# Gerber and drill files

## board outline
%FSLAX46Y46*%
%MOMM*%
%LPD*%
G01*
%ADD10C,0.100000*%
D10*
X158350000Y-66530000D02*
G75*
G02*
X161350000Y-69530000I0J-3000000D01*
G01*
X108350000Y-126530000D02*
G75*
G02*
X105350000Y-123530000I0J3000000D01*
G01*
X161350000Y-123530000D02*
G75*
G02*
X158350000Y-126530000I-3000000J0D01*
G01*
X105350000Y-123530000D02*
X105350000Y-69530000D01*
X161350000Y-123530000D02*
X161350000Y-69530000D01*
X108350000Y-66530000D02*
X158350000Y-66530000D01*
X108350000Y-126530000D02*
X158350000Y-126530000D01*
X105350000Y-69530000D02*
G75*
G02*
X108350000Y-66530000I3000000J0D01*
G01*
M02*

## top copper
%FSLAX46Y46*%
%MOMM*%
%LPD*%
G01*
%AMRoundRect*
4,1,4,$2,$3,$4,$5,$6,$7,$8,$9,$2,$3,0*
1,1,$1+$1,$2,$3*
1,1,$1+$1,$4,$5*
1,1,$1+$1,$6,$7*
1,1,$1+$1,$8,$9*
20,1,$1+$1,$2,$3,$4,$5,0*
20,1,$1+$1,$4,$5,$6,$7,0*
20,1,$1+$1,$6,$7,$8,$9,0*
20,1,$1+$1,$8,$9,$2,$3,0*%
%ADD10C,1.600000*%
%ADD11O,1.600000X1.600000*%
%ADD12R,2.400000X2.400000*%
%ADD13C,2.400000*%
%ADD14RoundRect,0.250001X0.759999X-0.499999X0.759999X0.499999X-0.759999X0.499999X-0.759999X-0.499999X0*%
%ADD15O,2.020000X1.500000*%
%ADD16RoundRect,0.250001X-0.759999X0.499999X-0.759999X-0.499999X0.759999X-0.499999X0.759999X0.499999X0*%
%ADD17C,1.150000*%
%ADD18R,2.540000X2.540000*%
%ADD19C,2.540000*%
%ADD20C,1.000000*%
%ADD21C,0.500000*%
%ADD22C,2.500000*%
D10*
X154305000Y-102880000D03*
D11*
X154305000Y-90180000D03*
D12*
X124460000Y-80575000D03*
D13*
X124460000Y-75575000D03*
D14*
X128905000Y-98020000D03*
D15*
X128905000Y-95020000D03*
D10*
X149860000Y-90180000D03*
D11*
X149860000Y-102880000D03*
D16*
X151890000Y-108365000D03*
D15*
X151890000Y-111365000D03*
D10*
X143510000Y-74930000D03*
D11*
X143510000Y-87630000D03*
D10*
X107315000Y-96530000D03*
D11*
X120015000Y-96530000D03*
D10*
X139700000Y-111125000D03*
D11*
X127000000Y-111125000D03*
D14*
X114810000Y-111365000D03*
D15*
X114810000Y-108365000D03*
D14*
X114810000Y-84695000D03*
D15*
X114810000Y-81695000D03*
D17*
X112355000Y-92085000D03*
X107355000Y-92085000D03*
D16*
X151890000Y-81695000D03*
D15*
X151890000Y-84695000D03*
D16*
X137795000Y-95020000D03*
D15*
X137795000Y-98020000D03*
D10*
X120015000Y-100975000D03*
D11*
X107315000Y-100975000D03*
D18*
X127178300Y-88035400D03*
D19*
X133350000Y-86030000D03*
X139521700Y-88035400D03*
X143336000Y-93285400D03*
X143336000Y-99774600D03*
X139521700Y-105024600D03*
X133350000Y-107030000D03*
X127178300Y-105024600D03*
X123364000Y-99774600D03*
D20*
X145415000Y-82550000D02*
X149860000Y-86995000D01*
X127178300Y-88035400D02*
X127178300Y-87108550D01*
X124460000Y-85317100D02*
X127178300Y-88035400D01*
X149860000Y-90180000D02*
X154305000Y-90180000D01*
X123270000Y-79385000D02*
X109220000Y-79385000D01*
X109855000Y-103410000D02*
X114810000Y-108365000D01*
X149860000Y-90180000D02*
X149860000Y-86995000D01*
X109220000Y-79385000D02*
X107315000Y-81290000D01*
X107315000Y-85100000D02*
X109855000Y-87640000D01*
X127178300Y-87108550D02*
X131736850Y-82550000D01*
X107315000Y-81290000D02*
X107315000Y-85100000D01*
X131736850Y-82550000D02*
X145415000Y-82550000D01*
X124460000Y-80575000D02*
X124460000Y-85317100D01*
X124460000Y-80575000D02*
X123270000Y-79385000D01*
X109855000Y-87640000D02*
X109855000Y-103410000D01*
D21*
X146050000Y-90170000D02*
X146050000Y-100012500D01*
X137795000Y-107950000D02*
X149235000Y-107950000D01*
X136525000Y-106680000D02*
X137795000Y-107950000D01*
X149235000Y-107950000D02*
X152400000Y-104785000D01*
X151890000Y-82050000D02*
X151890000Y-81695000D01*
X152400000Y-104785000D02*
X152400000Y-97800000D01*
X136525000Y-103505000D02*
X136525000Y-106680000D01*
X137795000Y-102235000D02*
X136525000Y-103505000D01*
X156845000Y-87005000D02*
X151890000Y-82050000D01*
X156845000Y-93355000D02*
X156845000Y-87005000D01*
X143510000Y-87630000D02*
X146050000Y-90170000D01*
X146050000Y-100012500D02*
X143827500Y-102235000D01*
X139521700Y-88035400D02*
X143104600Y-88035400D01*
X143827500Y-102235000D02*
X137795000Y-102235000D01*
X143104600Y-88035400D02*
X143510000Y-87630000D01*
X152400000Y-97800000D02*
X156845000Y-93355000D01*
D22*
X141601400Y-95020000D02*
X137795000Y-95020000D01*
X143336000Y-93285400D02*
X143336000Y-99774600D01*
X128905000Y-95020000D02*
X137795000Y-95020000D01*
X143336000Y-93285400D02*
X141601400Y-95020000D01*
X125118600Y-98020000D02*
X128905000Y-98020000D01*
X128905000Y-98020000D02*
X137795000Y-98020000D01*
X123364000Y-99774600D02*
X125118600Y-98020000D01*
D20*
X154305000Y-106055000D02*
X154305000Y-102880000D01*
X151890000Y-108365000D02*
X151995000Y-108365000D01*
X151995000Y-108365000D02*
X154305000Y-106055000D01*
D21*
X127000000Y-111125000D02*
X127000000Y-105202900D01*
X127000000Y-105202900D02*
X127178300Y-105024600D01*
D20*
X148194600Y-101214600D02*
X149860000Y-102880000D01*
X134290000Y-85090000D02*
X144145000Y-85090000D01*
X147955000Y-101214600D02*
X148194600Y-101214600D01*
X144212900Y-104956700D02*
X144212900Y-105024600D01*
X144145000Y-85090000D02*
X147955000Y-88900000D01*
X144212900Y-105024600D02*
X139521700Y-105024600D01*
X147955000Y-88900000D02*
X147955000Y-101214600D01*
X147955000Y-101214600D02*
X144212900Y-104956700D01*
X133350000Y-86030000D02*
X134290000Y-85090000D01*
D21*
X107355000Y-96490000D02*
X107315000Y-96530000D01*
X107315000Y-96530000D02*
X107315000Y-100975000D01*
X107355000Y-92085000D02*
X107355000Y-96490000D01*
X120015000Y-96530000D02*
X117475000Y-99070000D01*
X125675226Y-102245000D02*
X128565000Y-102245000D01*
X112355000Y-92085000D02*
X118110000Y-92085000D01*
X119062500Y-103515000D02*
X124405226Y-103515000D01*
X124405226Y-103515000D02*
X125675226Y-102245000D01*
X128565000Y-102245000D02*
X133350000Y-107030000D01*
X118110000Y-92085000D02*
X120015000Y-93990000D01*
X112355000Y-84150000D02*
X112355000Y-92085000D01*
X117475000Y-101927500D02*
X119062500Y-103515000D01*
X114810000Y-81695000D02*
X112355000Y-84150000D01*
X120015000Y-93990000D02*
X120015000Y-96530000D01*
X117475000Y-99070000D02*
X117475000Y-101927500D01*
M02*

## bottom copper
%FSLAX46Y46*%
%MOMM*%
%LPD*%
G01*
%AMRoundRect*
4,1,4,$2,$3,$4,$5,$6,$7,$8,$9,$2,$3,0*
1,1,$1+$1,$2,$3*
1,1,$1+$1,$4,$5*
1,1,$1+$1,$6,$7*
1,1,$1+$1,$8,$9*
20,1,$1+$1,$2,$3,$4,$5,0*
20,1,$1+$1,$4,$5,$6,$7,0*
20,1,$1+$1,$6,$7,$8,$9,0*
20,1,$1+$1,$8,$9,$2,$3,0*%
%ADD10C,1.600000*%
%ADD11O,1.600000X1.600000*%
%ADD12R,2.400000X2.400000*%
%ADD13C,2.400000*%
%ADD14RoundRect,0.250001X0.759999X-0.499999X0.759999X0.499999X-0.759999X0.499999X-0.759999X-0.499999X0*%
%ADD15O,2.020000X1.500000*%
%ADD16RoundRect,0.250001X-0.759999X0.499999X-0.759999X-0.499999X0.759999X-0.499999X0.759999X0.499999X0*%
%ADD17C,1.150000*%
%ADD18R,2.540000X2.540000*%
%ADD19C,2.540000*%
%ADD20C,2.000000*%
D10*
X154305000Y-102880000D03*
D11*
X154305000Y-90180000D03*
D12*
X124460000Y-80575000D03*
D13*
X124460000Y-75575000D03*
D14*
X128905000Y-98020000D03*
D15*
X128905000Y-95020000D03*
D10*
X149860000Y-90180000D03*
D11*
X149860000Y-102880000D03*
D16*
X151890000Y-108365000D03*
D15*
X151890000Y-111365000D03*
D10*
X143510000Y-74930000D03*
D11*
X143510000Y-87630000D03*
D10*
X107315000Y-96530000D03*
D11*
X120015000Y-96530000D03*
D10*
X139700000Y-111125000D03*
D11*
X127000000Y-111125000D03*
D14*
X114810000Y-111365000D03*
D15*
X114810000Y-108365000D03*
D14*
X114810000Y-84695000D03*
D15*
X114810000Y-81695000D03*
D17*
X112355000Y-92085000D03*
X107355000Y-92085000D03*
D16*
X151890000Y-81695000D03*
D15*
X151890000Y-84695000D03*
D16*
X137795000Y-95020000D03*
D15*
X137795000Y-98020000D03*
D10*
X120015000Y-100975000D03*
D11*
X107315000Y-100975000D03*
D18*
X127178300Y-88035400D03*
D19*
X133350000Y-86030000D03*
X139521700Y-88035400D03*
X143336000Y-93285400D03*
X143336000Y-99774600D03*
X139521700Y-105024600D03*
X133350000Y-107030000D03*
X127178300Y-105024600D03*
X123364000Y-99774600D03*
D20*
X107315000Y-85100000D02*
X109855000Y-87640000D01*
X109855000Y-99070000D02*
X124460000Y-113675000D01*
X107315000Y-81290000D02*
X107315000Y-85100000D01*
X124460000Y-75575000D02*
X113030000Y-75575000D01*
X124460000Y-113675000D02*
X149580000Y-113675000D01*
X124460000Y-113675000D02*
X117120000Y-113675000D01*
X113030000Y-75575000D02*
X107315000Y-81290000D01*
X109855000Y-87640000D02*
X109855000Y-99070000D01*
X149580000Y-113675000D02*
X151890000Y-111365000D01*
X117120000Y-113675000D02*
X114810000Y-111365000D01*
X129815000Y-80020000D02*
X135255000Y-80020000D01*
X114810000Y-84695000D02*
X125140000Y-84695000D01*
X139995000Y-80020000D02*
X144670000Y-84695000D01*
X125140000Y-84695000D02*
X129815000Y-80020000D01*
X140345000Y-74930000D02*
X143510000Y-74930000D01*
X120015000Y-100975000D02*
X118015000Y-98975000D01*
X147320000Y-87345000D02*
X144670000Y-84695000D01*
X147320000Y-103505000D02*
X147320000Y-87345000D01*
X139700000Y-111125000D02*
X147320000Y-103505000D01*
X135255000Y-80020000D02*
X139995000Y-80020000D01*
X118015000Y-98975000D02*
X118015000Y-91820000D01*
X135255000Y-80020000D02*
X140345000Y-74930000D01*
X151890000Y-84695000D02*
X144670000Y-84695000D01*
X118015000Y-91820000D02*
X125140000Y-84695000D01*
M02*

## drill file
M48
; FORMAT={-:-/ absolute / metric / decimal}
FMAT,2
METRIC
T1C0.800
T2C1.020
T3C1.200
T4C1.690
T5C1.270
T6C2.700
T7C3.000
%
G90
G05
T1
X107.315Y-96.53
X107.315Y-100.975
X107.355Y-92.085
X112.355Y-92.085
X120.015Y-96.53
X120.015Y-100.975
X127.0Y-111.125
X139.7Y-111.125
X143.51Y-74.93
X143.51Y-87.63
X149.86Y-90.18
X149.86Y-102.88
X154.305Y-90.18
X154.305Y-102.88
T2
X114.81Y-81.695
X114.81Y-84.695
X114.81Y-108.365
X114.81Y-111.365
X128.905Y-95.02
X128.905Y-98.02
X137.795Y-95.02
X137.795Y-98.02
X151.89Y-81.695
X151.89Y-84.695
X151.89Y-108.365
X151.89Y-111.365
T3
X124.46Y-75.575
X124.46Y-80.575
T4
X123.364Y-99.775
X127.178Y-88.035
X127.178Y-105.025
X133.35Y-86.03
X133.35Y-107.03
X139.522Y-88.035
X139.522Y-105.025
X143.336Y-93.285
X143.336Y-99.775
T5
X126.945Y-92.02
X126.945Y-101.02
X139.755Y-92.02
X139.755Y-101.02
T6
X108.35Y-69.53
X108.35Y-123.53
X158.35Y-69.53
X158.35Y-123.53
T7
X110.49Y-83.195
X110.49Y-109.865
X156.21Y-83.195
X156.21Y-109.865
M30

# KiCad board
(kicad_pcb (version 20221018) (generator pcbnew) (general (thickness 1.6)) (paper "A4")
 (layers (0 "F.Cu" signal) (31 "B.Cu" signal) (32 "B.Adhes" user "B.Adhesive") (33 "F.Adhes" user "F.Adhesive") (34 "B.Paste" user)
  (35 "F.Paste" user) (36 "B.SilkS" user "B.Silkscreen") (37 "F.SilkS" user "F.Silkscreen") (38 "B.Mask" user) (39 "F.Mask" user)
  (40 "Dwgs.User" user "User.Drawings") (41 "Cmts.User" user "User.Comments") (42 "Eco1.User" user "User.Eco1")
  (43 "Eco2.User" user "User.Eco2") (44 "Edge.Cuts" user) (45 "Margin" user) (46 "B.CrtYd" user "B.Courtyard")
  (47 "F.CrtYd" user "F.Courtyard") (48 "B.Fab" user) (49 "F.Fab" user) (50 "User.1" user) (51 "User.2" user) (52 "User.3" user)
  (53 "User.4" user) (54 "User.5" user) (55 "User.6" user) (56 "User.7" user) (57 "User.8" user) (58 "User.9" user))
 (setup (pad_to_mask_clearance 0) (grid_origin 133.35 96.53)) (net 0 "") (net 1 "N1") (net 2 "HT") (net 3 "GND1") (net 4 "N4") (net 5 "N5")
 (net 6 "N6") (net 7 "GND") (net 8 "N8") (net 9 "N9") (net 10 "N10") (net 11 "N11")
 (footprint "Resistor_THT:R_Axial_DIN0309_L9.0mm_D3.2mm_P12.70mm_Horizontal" (layer "F.Cu") (at 154.305 102.88 90)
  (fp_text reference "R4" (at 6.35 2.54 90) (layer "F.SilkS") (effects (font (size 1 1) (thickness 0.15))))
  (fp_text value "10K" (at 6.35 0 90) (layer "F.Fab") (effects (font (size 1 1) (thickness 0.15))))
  (pad "1" thru_hole circle (at 0 0 90) (size 1.6 1.6) (drill 0.8) (layers "*.Cu" "*.Mask") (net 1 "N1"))
  (pad "2" thru_hole oval (at 12.7 0 90) (size 1.6 1.6) (drill 0.8) (layers "*.Cu" "*.Mask") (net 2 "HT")))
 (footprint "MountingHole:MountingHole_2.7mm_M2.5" (layer "F.Cu") (at 158.35 69.53)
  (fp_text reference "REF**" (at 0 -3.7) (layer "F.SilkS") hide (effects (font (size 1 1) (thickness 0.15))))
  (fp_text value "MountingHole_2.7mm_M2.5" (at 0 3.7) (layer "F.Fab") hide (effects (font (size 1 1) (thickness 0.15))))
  (pad "" np_thru_hole circle (at 0 0) (size 2.7 2.7) (drill 2.7) (layers "*.Cu" "*.Mask")))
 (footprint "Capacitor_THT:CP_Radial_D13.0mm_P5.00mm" (layer "F.Cu") (at 124.46 80.575 90)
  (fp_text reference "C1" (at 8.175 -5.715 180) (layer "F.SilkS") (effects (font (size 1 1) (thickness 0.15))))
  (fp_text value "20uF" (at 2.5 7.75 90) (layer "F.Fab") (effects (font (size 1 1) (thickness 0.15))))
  (pad "1" thru_hole rect (at 0 0 90) (size 2.4 2.4) (drill 1.2) (layers "*.Cu" "*.Mask") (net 2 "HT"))
  (pad "2" thru_hole circle (at 5 0 90) (size 2.4 2.4) (drill 1.2) (layers "*.Cu" "*.Mask") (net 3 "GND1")))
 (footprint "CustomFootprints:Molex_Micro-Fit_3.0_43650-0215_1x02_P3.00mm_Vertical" (layer "F.Cu") (at 128.905 98.02 90)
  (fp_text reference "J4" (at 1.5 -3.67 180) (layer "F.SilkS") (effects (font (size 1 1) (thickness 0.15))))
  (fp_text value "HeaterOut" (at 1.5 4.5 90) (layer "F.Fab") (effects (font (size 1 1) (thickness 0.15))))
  (pad "" np_thru_hole circle (at -3 -1.96 90) (size 1.27 1.27) (drill 1.27) (layers "*.Cu" "*.Mask"))
  (pad "" np_thru_hole circle (at 6 -1.96 90) (size 1.27 1.27) (drill 1.27) (layers "*.Cu" "*.Mask"))
  (pad "1" thru_hole roundrect (at 0 0 90) (size 1.5 2.02) (drill 1.02) (layers "*.Cu" "*.Mask") (roundrect_rratio 0.166667) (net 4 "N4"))
  (pad "2" thru_hole oval (at 3 0 90) (size 1.5 2.02) (drill 1.02) (layers "*.Cu" "*.Mask") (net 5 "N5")))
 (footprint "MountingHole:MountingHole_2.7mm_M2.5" (layer "F.Cu") (at 108.35 123.53)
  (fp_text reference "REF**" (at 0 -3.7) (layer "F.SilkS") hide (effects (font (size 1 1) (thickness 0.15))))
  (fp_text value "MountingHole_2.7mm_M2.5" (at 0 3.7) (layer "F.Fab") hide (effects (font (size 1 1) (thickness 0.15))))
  (pad "" np_thru_hole circle (at 0 0) (size 2.7 2.7) (drill 2.7) (layers "*.Cu" "*.Mask")))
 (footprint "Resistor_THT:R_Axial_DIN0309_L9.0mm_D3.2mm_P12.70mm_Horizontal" (layer "F.Cu") (at 149.86 90.18 -90)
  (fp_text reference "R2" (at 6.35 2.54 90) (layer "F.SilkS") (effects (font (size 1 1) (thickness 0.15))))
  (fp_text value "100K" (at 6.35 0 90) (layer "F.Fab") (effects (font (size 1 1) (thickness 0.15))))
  (pad "1" thru_hole circle (at 0 0 270) (size 1.6 1.6) (drill 0.8) (layers "*.Cu" "*.Mask") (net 2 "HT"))
  (pad "2" thru_hole oval (at 12.7 0 270) (size 1.6 1.6) (drill 0.8) (layers "*.Cu" "*.Mask") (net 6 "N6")))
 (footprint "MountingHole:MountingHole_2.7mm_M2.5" (layer "F.Cu") (at 158.35 123.53)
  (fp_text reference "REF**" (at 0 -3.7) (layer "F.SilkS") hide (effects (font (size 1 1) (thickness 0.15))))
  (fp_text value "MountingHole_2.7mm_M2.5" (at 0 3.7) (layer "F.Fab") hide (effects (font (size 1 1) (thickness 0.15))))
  (pad "" np_thru_hole circle (at 0 0) (size 2.7 2.7) (drill 2.7) (layers "*.Cu" "*.Mask")))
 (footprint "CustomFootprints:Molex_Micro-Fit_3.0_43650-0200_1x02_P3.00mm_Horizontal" (layer "F.Cu") (at 151.89 108.365 -90)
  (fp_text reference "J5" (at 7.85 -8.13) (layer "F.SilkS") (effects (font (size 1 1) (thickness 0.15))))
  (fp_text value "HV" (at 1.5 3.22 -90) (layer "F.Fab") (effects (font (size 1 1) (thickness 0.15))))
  (pad "" np_thru_hole circle (at 1.5 -4.32 270) (size 3 3) (drill 3) (layers "*.Cu" "*.Mask"))
  (pad "1" thru_hole roundrect (at 0 0 270) (size 1.5 2.02) (drill 1.02) (layers "*.Cu" "*.Mask") (roundrect_rratio 0.166667) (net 1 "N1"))
  (pad "2" thru_hole oval (at 3 0 270) (size 1.5 2.02) (drill 1.02) (layers "*.Cu" "*.Mask") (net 3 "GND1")))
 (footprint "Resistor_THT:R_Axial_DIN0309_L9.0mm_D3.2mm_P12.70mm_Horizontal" (layer "F.Cu") (at 143.51 74.93 -90)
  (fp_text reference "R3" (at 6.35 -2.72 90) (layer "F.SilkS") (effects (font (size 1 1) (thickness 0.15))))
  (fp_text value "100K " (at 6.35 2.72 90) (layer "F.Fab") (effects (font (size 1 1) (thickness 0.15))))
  (pad "1" thru_hole circle (at 0 0 270) (size 1.6 1.6) (drill 0.8) (layers "*.Cu" "*.Mask") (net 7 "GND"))
  (pad "2" thru_hole oval (at 12.7 0 270) (size 1.6 1.6) (drill 0.8) (layers "*.Cu" "*.Mask") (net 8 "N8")))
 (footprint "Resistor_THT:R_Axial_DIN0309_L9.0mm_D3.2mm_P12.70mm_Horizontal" (layer "F.Cu") (at 107.315 96.53)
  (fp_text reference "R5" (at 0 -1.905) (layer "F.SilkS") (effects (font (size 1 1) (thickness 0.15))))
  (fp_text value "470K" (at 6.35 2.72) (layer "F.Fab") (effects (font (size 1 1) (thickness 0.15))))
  (pad "1" thru_hole circle (at 0 0) (size 1.6 1.6) (drill 0.8) (layers "*.Cu" "*.Mask") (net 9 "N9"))
  (pad "2" thru_hole oval (at 12.7 0) (size 1.6 1.6) (drill 0.8) (layers "*.Cu" "*.Mask") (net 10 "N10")))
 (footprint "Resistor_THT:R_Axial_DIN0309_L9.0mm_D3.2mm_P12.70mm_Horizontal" (layer "F.Cu") (at 139.7 111.125 180)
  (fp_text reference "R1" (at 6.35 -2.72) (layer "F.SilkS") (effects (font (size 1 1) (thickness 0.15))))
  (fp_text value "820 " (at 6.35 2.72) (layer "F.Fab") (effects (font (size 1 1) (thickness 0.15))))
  (pad "1" thru_hole circle (at 0 0 180) (size 1.6 1.6) (drill 0.8) (layers "*.Cu" "*.Mask") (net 7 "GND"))
  (pad "2" thru_hole oval (at 12.7 0 180) (size 1.6 1.6) (drill 0.8) (layers "*.Cu" "*.Mask") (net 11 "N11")))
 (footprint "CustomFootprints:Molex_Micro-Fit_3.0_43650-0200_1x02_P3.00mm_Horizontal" (layer "F.Cu") (at 114.81 111.365 90)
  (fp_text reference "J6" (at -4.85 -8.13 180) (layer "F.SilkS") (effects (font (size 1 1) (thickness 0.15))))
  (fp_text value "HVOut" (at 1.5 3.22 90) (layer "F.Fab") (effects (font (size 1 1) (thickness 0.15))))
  (pad "" np_thru_hole circle (at 1.5 -4.32 90) (size 3 3) (drill 3) (layers "*.Cu" "*.Mask"))
  (pad "1" thru_hole roundrect (at 0 0 90) (size 1.5 2.02) (drill 1.02) (layers "*.Cu" "*.Mask") (roundrect_rratio 0.166667) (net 3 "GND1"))
  (pad "2" thru_hole oval (at 3 0 90) (size 1.5 2.02) (drill 1.02) (layers "*.Cu" "*.Mask") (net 2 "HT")))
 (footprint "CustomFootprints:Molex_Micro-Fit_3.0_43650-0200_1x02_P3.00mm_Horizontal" (layer "F.Cu") (at 114.81 84.695 90)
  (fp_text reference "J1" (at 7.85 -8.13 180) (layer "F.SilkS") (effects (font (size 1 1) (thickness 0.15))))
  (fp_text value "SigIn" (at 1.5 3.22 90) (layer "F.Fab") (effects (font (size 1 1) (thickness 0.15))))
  (pad "" np_thru_hole circle (at 1.5 -4.32 90) (size 3 3) (drill 3) (layers "*.Cu" "*.Mask"))
  (pad "1" thru_hole roundrect (at 0 0 90) (size 1.5 2.02) (drill 1.02) (layers "*.Cu" "*.Mask") (roundrect_rratio 0.166667) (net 7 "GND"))
  (pad "2" thru_hole oval (at 3 0 90) (size 1.5 2.02) (drill 1.02) (layers "*.Cu" "*.Mask") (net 10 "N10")))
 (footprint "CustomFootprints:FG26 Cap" (layer "F.Cu") (at 109.855 92.085 180)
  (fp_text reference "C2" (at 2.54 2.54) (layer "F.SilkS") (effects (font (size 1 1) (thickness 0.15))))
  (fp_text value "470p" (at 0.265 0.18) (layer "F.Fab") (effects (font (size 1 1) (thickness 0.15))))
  (pad "1" thru_hole circle (at -2.5 0 180) (size 1.15 1.15) (drill 0.8) (layers "*.Cu" "*.Mask") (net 10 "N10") (solder_mask_margin 0.102))
  (pad "2" thru_hole circle (at 2.5 0 180) (size 1.15 1.15) (drill 0.8) (layers "*.Cu" "*.Mask") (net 9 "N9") (solder_mask_margin 0.102)))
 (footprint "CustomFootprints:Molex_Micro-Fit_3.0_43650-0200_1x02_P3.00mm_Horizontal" (layer "F.Cu") (at 151.89 81.695 -90)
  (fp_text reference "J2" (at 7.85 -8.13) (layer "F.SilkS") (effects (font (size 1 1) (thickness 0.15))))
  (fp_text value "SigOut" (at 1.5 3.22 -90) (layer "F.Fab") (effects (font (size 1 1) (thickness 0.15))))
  (pad "" np_thru_hole circle (at 1.5 -4.32 270) (size 3 3) (drill 3) (layers "*.Cu" "*.Mask"))
  (pad "1" thru_hole roundrect (at 0 0 270) (size 1.5 2.02) (drill 1.02) (layers "*.Cu" "*.Mask") (roundrect_rratio 0.166667) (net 8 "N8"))
  (pad "2" thru_hole oval (at 3 0 270) (size 1.5 2.02) (drill 1.02) (layers "*.Cu" "*.Mask") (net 7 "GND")))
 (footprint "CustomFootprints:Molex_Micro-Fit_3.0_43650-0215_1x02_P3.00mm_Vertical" (layer "F.Cu") (at 137.795 95.02 -90)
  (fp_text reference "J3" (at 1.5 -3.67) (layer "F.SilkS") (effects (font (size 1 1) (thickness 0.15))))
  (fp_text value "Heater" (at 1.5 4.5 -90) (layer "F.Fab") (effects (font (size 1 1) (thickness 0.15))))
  (pad "" np_thru_hole circle (at -3 -1.96 270) (size 1.27 1.27) (drill 1.27) (layers "*.Cu" "*.Mask"))
  (pad "" np_thru_hole circle (at 6 -1.96 270) (size 1.27 1.27) (drill 1.27) (layers "*.Cu" "*.Mask"))
  (pad "1" thru_hole roundrect (at 0 0 270) (size 1.5 2.02) (drill 1.02) (layers "*.Cu" "*.Mask") (roundrect_rratio 0.166667) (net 5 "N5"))
  (pad "2" thru_hole oval (at 3 0 270) (size 1.5 2.02) (drill 1.02) (layers "*.Cu" "*.Mask") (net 4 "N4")))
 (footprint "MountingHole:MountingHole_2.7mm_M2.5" (layer "F.Cu") (at 108.35 69.53)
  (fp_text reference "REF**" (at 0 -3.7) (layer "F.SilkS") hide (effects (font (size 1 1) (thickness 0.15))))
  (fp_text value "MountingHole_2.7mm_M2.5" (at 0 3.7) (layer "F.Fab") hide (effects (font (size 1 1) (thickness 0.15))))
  (pad "" np_thru_hole circle (at 0 0) (size 2.7 2.7) (drill 2.7) (layers "*.Cu" "*.Mask")))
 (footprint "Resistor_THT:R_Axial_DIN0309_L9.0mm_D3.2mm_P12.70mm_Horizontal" (layer "F.Cu") (at 120.015 100.975 180)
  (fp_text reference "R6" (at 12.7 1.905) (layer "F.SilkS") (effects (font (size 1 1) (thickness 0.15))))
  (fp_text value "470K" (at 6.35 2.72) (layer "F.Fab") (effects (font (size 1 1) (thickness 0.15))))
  (pad "1" thru_hole circle (at 0 0 180) (size 1.6 1.6) (drill 0.8) (layers "*.Cu" "*.Mask") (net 7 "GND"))
  (pad "2" thru_hole oval (at 12.7 0 180) (size 1.6 1.6) (drill 0.8) (layers "*.Cu" "*.Mask") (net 9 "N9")))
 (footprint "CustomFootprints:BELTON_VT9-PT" (layer "B.Cu") (at 133.35 96.53 180)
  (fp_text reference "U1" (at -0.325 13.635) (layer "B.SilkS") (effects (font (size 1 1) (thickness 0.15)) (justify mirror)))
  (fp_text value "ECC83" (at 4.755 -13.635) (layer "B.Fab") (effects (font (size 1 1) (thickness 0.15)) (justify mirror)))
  (pad "1" thru_hole rect (at 6.1717 8.4946 180) (size 2.54 2.54) (drill 1.69) (layers "*.Cu" "*.Mask") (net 2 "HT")
   (solder_mask_margin 0.102))
  (pad "2" thru_hole circle (at 0 10.5 180) (size 2.54 2.54) (drill 1.69) (layers "*.Cu" "*.Mask") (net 6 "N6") (solder_mask_margin 0.102))
  (pad "3" thru_hole circle (at -6.1717 8.4946 180) (size 2.54 2.54) (drill 1.69) (layers "*.Cu" "*.Mask") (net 8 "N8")
   (solder_mask_margin 0.102))
  (pad "4" thru_hole circle (at -9.986 3.2446 180) (size 2.54 2.54) (drill 1.69) (layers "*.Cu" "*.Mask") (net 5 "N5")
   (solder_mask_margin 0.102))
  (pad "5" thru_hole circle (at -9.986 -3.2446 180) (size 2.54 2.54) (drill 1.69) (layers "*.Cu" "*.Mask") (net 5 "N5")
   (solder_mask_margin 0.102))
  (pad "6" thru_hole circle (at -6.1717 -8.4946 180) (size 2.54 2.54) (drill 1.69) (layers "*.Cu" "*.Mask") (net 6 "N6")
   (solder_mask_margin 0.102))
  (pad "7" thru_hole circle (at 0 -10.5 180) (size 2.54 2.54) (drill 1.69) (layers "*.Cu" "*.Mask") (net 10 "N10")
   (solder_mask_margin 0.102))
  (pad "8" thru_hole circle (at 6.1717 -8.4946 180) (size 2.54 2.54) (drill 1.69) (layers "*.Cu" "*.Mask") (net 11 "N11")
   (solder_mask_margin 0.102))
  (pad "9" thru_hole circle (at 9.986 -3.2446 180) (size 2.54 2.54) (drill 1.69) (layers "*.Cu" "*.Mask") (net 4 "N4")
   (solder_mask_margin 0.102)))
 (gr_arc (start 158.35 66.53) (mid 160.47132 67.40868) (end 161.35 69.53) (stroke (width 0.1) (type default)) (layer "Edge.Cuts"))
 (gr_arc (start 108.35 126.53) (mid 106.22868 125.65132) (end 105.35 123.53) (stroke (width 0.1) (type default)) (layer "Edge.Cuts"))
 (gr_arc (start 161.35 123.53) (mid 160.47132 125.65132) (end 158.35 126.53) (stroke (width 0.1) (type default)) (layer "Edge.Cuts"))
 (gr_line (start 105.35 123.53) (end 105.35 69.53) (stroke (width 0.1) (type default)) (layer "Edge.Cuts"))
 (gr_line (start 161.35 123.53) (end 161.35 69.53) (stroke (width 0.1) (type default)) (layer "Edge.Cuts"))
 (gr_line (start 108.35 66.53) (end 158.35 66.53) (stroke (width 0.1) (type default)) (layer "Edge.Cuts"))
 (gr_line (start 108.35 126.53) (end 158.35 126.53) (stroke (width 0.1) (type default)) (layer "Edge.Cuts"))
 (gr_arc (start 105.35 69.53) (mid 106.22868 67.40868) (end 108.35 66.53) (stroke (width 0.1) (type default)) (layer "Edge.Cuts"))
 (segment (start 145.415 82.55) (end 149.86 86.995) (width 1) (layer "F.Cu") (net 2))
 (segment (start 127.1783 88.0354) (end 127.1783 87.10855) (width 1) (layer "F.Cu") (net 2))
 (segment (start 124.46 85.3171) (end 127.1783 88.0354) (width 1) (layer "F.Cu") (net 2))
 (segment (start 149.86 90.18) (end 154.305 90.18) (width 1) (layer "F.Cu") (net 2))
 (segment (start 123.27 79.385) (end 109.22 79.385) (width 1) (layer "F.Cu") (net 2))
 (segment (start 109.855 103.41) (end 114.81 108.365) (width 1) (layer "F.Cu") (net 2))
 (segment (start 149.86 90.18) (end 149.86 86.995) (width 1) (layer "F.Cu") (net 2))
 (segment (start 109.22 79.385) (end 107.315 81.29) (width 1) (layer "F.Cu") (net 2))
 (segment (start 107.315 85.1) (end 109.855 87.64) (width 1) (layer "F.Cu") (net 2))
 (segment (start 127.1783 87.10855) (end 131.73685 82.55) (width 1) (layer "F.Cu") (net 2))
 (segment (start 107.315 81.29) (end 107.315 85.1) (width 1) (layer "F.Cu") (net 2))
 (segment (start 131.73685 82.55) (end 145.415 82.55) (width 1) (layer "F.Cu") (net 2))
 (segment (start 124.46 80.575) (end 124.46 85.3171) (width 1) (layer "F.Cu") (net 2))
 (segment (start 124.46 80.575) (end 123.27 79.385) (width 1) (layer "F.Cu") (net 2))
 (segment (start 109.855 87.64) (end 109.855 103.41) (width 1) (layer "F.Cu") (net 2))
 (segment (start 107.315 85.1) (end 109.855 87.64) (width 2) (layer "B.Cu") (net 3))
 (segment (start 109.855 99.07) (end 124.46 113.675) (width 2) (layer "B.Cu") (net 3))
 (segment (start 107.315 81.29) (end 107.315 85.1) (width 2) (layer "B.Cu") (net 3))
 (segment (start 124.46 75.575) (end 113.03 75.575) (width 2) (layer "B.Cu") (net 3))
 (segment (start 124.46 113.675) (end 149.58 113.675) (width 2) (layer "B.Cu") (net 3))
 (segment (start 124.46 113.675) (end 117.12 113.675) (width 2) (layer "B.Cu") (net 3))
 (segment (start 113.03 75.575) (end 107.315 81.29) (width 2) (layer "B.Cu") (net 3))
 (segment (start 109.855 87.64) (end 109.855 99.07) (width 2) (layer "B.Cu") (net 3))
 (segment (start 149.58 113.675) (end 151.89 111.365) (width 2) (layer "B.Cu") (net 3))
 (segment (start 117.12 113.675) (end 114.81 111.365) (width 2) (layer "B.Cu") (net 3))
 (segment (start 129.815 80.02) (end 135.255 80.02) (width 2) (layer "B.Cu") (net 7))
 (segment (start 114.81 84.695) (end 125.14 84.695) (width 2) (layer "B.Cu") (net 7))
 (segment (start 139.995 80.02) (end 144.67 84.695) (width 2) (layer "B.Cu") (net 7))
 (segment (start 125.14 84.695) (end 129.815 80.02) (width 2) (layer "B.Cu") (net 7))
 (segment (start 140.345 74.93) (end 143.51 74.93) (width 2) (layer "B.Cu") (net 7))
 (segment (start 120.015 100.975) (end 118.015 98.975) (width 2) (layer "B.Cu") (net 7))
 (segment (start 147.32 87.345) (end 144.67 84.695) (width 2) (layer "B.Cu") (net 7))
 (segment (start 147.32 103.505) (end 147.32 87.345) (width 2) (layer "B.Cu") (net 7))
 (segment (start 139.7 111.125) (end 147.32 103.505) (width 2) (layer "B.Cu") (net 7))
 (segment (start 135.255 80.02) (end 139.995 80.02) (width 2) (layer "B.Cu") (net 7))
 (segment (start 118.015 98.975) (end 118.015 91.82) (width 2) (layer "B.Cu") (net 7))
 (segment (start 135.255 80.02) (end 140.345 74.93) (width 2) (layer "B.Cu") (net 7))
 (segment (start 151.89 84.695) (end 144.67 84.695) (width 2) (layer "B.Cu") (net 7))
 (segment (start 118.015 91.82) (end 125.14 84.695) (width 2) (layer "B.Cu") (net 7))
 (segment (start 146.05 90.17) (end 146.05 100.0125) (width 0.5) (layer "F.Cu") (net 8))
 (segment (start 137.795 107.95) (end 149.235 107.95) (width 0.5) (layer "F.Cu") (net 8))
 (segment (start 136.525 106.68) (end 137.795 107.95) (width 0.5) (layer "F.Cu") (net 8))
 (segment (start 149.235 107.95) (end 152.4 104.785) (width 0.5) (layer "F.Cu") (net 8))
 (segment (start 151.89 82.05) (end 151.89 81.695) (width 0.5) (layer "F.Cu") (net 8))
 (segment (start 152.4 104.785) (end 152.4 97.8) (width 0.5) (layer "F.Cu") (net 8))
 (segment (start 136.525 103.505) (end 136.525 106.68) (width 0.5) (layer "F.Cu") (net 8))
 (segment (start 137.795 102.235) (end 136.525 103.505) (width 0.5) (layer "F.Cu") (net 8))
 (segment (start 156.845 87.005) (end 151.89 82.05) (width 0.5) (layer "F.Cu") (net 8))
 (segment (start 156.845 93.355) (end 156.845 87.005) (width 0.5) (layer "F.Cu") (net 8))
 (segment (start 143.51 87.63) (end 146.05 90.17) (width 0.5) (layer "F.Cu") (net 8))
 (segment (start 146.05 100.0125) (end 143.8275 102.235) (width 0.5) (layer "F.Cu") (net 8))
 (segment (start 139.5217 88.0354) (end 143.1046 88.0354) (width 0.5) (layer "F.Cu") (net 8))
 (segment (start 143.8275 102.235) (end 137.795 102.235) (width 0.5) (layer "F.Cu") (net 8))
 (segment (start 143.1046 88.0354) (end 143.51 87.63) (width 0.5) (layer "F.Cu") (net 8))
 (segment (start 152.4 97.8) (end 156.845 93.355) (width 0.5) (layer "F.Cu") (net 8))
 (segment (start 141.6014 95.02) (end 137.795 95.02) (width 2.5) (layer "F.Cu") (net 5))
 (segment (start 143.336 93.2854) (end 143.336 99.7746) (width 2.5) (layer "F.Cu") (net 5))
 (segment (start 128.905 95.02) (end 137.795 95.02) (width 2.5) (layer "F.Cu") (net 5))
 (segment (start 143.336 93.2854) (end 141.6014 95.02) (width 2.5) (layer "F.Cu") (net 5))
 (segment (start 125.1186 98.02) (end 128.905 98.02) (width 2.5) (layer "F.Cu") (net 4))
 (segment (start 128.905 98.02) (end 137.795 98.02) (width 2.5) (layer "F.Cu") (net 4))
 (segment (start 123.364 99.7746) (end 125.1186 98.02) (width 2.5) (layer "F.Cu") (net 4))
 (segment (start 154.305 106.055) (end 154.305 102.88) (width 1) (layer "F.Cu") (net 1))
 (segment (start 151.89 108.365) (end 151.995 108.365) (width 1) (layer "F.Cu") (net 1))
 (segment (start 151.995 108.365) (end 154.305 106.055) (width 1) (layer "F.Cu") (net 1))
 (segment (start 127 111.125) (end 127 105.2029) (width 0.5) (layer "F.Cu") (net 11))
 (segment (start 127 105.2029) (end 127.1783 105.0246) (width 0.5) (layer "F.Cu") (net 11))
 (segment (start 148.1946 101.2146) (end 149.86 102.88) (width 1) (layer "F.Cu") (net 6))
 (segment (start 134.29 85.09) (end 144.145 85.09) (width 1) (layer "F.Cu") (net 6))
 (segment (start 147.955 101.2146) (end 148.1946 101.2146) (width 1) (layer "F.Cu") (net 6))
 (segment (start 144.2129 104.9567) (end 144.2129 105.0246) (width 1) (layer "F.Cu") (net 6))
 (segment (start 144.145 85.09) (end 147.955 88.9) (width 1) (layer "F.Cu") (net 6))
 (segment (start 144.2129 105.0246) (end 139.5217 105.0246) (width 1) (layer "F.Cu") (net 6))
 (segment (start 147.955 88.9) (end 147.955 101.2146) (width 1) (layer "F.Cu") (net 6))
 (segment (start 147.955 101.2146) (end 144.2129 104.9567) (width 1) (layer "F.Cu") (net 6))
 (segment (start 133.35 86.03) (end 134.29 85.09) (width 1) (layer "F.Cu") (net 6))
 (segment (start 107.355 96.49) (end 107.315 96.53) (width 0.5) (layer "F.Cu") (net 9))
 (segment (start 107.315 96.53) (end 107.315 100.975) (width 0.5) (layer "F.Cu") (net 9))
 (segment (start 107.355 92.085) (end 107.355 96.49) (width 0.5) (layer "F.Cu") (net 9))
 (segment (start 120.015 96.53) (end 117.475 99.07) (width 0.5) (layer "F.Cu") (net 10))
 (segment (start 125.675226 102.245) (end 128.565 102.245) (width 0.5) (layer "F.Cu") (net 10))
 (segment (start 112.355 92.085) (end 118.11 92.085) (width 0.5) (layer "F.Cu") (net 10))
 (segment (start 119.0625 103.515) (end 124.405226 103.515) (width 0.5) (layer "F.Cu") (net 10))
 (segment (start 124.405226 103.515) (end 125.675226 102.245) (width 0.5) (layer "F.Cu") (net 10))
 (segment (start 128.565 102.245) (end 133.35 107.03) (width 0.5) (layer "F.Cu") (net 10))
 (segment (start 118.11 92.085) (end 120.015 93.99) (width 0.5) (layer "F.Cu") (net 10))
 (segment (start 112.355 84.15) (end 112.355 92.085) (width 0.5) (layer "F.Cu") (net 10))
 (segment (start 117.475 101.9275) (end 119.0625 103.515) (width 0.5) (layer "F.Cu") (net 10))
 (segment (start 114.81 81.695) (end 112.355 84.15) (width 0.5) (layer "F.Cu") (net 10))
 (segment (start 120.015 93.99) (end 120.015 96.53) (width 0.5) (layer "F.Cu") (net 10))
 (segment (start 117.475 99.07) (end 117.475 101.9275) (width 0.5) (layer "F.Cu") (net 10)))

